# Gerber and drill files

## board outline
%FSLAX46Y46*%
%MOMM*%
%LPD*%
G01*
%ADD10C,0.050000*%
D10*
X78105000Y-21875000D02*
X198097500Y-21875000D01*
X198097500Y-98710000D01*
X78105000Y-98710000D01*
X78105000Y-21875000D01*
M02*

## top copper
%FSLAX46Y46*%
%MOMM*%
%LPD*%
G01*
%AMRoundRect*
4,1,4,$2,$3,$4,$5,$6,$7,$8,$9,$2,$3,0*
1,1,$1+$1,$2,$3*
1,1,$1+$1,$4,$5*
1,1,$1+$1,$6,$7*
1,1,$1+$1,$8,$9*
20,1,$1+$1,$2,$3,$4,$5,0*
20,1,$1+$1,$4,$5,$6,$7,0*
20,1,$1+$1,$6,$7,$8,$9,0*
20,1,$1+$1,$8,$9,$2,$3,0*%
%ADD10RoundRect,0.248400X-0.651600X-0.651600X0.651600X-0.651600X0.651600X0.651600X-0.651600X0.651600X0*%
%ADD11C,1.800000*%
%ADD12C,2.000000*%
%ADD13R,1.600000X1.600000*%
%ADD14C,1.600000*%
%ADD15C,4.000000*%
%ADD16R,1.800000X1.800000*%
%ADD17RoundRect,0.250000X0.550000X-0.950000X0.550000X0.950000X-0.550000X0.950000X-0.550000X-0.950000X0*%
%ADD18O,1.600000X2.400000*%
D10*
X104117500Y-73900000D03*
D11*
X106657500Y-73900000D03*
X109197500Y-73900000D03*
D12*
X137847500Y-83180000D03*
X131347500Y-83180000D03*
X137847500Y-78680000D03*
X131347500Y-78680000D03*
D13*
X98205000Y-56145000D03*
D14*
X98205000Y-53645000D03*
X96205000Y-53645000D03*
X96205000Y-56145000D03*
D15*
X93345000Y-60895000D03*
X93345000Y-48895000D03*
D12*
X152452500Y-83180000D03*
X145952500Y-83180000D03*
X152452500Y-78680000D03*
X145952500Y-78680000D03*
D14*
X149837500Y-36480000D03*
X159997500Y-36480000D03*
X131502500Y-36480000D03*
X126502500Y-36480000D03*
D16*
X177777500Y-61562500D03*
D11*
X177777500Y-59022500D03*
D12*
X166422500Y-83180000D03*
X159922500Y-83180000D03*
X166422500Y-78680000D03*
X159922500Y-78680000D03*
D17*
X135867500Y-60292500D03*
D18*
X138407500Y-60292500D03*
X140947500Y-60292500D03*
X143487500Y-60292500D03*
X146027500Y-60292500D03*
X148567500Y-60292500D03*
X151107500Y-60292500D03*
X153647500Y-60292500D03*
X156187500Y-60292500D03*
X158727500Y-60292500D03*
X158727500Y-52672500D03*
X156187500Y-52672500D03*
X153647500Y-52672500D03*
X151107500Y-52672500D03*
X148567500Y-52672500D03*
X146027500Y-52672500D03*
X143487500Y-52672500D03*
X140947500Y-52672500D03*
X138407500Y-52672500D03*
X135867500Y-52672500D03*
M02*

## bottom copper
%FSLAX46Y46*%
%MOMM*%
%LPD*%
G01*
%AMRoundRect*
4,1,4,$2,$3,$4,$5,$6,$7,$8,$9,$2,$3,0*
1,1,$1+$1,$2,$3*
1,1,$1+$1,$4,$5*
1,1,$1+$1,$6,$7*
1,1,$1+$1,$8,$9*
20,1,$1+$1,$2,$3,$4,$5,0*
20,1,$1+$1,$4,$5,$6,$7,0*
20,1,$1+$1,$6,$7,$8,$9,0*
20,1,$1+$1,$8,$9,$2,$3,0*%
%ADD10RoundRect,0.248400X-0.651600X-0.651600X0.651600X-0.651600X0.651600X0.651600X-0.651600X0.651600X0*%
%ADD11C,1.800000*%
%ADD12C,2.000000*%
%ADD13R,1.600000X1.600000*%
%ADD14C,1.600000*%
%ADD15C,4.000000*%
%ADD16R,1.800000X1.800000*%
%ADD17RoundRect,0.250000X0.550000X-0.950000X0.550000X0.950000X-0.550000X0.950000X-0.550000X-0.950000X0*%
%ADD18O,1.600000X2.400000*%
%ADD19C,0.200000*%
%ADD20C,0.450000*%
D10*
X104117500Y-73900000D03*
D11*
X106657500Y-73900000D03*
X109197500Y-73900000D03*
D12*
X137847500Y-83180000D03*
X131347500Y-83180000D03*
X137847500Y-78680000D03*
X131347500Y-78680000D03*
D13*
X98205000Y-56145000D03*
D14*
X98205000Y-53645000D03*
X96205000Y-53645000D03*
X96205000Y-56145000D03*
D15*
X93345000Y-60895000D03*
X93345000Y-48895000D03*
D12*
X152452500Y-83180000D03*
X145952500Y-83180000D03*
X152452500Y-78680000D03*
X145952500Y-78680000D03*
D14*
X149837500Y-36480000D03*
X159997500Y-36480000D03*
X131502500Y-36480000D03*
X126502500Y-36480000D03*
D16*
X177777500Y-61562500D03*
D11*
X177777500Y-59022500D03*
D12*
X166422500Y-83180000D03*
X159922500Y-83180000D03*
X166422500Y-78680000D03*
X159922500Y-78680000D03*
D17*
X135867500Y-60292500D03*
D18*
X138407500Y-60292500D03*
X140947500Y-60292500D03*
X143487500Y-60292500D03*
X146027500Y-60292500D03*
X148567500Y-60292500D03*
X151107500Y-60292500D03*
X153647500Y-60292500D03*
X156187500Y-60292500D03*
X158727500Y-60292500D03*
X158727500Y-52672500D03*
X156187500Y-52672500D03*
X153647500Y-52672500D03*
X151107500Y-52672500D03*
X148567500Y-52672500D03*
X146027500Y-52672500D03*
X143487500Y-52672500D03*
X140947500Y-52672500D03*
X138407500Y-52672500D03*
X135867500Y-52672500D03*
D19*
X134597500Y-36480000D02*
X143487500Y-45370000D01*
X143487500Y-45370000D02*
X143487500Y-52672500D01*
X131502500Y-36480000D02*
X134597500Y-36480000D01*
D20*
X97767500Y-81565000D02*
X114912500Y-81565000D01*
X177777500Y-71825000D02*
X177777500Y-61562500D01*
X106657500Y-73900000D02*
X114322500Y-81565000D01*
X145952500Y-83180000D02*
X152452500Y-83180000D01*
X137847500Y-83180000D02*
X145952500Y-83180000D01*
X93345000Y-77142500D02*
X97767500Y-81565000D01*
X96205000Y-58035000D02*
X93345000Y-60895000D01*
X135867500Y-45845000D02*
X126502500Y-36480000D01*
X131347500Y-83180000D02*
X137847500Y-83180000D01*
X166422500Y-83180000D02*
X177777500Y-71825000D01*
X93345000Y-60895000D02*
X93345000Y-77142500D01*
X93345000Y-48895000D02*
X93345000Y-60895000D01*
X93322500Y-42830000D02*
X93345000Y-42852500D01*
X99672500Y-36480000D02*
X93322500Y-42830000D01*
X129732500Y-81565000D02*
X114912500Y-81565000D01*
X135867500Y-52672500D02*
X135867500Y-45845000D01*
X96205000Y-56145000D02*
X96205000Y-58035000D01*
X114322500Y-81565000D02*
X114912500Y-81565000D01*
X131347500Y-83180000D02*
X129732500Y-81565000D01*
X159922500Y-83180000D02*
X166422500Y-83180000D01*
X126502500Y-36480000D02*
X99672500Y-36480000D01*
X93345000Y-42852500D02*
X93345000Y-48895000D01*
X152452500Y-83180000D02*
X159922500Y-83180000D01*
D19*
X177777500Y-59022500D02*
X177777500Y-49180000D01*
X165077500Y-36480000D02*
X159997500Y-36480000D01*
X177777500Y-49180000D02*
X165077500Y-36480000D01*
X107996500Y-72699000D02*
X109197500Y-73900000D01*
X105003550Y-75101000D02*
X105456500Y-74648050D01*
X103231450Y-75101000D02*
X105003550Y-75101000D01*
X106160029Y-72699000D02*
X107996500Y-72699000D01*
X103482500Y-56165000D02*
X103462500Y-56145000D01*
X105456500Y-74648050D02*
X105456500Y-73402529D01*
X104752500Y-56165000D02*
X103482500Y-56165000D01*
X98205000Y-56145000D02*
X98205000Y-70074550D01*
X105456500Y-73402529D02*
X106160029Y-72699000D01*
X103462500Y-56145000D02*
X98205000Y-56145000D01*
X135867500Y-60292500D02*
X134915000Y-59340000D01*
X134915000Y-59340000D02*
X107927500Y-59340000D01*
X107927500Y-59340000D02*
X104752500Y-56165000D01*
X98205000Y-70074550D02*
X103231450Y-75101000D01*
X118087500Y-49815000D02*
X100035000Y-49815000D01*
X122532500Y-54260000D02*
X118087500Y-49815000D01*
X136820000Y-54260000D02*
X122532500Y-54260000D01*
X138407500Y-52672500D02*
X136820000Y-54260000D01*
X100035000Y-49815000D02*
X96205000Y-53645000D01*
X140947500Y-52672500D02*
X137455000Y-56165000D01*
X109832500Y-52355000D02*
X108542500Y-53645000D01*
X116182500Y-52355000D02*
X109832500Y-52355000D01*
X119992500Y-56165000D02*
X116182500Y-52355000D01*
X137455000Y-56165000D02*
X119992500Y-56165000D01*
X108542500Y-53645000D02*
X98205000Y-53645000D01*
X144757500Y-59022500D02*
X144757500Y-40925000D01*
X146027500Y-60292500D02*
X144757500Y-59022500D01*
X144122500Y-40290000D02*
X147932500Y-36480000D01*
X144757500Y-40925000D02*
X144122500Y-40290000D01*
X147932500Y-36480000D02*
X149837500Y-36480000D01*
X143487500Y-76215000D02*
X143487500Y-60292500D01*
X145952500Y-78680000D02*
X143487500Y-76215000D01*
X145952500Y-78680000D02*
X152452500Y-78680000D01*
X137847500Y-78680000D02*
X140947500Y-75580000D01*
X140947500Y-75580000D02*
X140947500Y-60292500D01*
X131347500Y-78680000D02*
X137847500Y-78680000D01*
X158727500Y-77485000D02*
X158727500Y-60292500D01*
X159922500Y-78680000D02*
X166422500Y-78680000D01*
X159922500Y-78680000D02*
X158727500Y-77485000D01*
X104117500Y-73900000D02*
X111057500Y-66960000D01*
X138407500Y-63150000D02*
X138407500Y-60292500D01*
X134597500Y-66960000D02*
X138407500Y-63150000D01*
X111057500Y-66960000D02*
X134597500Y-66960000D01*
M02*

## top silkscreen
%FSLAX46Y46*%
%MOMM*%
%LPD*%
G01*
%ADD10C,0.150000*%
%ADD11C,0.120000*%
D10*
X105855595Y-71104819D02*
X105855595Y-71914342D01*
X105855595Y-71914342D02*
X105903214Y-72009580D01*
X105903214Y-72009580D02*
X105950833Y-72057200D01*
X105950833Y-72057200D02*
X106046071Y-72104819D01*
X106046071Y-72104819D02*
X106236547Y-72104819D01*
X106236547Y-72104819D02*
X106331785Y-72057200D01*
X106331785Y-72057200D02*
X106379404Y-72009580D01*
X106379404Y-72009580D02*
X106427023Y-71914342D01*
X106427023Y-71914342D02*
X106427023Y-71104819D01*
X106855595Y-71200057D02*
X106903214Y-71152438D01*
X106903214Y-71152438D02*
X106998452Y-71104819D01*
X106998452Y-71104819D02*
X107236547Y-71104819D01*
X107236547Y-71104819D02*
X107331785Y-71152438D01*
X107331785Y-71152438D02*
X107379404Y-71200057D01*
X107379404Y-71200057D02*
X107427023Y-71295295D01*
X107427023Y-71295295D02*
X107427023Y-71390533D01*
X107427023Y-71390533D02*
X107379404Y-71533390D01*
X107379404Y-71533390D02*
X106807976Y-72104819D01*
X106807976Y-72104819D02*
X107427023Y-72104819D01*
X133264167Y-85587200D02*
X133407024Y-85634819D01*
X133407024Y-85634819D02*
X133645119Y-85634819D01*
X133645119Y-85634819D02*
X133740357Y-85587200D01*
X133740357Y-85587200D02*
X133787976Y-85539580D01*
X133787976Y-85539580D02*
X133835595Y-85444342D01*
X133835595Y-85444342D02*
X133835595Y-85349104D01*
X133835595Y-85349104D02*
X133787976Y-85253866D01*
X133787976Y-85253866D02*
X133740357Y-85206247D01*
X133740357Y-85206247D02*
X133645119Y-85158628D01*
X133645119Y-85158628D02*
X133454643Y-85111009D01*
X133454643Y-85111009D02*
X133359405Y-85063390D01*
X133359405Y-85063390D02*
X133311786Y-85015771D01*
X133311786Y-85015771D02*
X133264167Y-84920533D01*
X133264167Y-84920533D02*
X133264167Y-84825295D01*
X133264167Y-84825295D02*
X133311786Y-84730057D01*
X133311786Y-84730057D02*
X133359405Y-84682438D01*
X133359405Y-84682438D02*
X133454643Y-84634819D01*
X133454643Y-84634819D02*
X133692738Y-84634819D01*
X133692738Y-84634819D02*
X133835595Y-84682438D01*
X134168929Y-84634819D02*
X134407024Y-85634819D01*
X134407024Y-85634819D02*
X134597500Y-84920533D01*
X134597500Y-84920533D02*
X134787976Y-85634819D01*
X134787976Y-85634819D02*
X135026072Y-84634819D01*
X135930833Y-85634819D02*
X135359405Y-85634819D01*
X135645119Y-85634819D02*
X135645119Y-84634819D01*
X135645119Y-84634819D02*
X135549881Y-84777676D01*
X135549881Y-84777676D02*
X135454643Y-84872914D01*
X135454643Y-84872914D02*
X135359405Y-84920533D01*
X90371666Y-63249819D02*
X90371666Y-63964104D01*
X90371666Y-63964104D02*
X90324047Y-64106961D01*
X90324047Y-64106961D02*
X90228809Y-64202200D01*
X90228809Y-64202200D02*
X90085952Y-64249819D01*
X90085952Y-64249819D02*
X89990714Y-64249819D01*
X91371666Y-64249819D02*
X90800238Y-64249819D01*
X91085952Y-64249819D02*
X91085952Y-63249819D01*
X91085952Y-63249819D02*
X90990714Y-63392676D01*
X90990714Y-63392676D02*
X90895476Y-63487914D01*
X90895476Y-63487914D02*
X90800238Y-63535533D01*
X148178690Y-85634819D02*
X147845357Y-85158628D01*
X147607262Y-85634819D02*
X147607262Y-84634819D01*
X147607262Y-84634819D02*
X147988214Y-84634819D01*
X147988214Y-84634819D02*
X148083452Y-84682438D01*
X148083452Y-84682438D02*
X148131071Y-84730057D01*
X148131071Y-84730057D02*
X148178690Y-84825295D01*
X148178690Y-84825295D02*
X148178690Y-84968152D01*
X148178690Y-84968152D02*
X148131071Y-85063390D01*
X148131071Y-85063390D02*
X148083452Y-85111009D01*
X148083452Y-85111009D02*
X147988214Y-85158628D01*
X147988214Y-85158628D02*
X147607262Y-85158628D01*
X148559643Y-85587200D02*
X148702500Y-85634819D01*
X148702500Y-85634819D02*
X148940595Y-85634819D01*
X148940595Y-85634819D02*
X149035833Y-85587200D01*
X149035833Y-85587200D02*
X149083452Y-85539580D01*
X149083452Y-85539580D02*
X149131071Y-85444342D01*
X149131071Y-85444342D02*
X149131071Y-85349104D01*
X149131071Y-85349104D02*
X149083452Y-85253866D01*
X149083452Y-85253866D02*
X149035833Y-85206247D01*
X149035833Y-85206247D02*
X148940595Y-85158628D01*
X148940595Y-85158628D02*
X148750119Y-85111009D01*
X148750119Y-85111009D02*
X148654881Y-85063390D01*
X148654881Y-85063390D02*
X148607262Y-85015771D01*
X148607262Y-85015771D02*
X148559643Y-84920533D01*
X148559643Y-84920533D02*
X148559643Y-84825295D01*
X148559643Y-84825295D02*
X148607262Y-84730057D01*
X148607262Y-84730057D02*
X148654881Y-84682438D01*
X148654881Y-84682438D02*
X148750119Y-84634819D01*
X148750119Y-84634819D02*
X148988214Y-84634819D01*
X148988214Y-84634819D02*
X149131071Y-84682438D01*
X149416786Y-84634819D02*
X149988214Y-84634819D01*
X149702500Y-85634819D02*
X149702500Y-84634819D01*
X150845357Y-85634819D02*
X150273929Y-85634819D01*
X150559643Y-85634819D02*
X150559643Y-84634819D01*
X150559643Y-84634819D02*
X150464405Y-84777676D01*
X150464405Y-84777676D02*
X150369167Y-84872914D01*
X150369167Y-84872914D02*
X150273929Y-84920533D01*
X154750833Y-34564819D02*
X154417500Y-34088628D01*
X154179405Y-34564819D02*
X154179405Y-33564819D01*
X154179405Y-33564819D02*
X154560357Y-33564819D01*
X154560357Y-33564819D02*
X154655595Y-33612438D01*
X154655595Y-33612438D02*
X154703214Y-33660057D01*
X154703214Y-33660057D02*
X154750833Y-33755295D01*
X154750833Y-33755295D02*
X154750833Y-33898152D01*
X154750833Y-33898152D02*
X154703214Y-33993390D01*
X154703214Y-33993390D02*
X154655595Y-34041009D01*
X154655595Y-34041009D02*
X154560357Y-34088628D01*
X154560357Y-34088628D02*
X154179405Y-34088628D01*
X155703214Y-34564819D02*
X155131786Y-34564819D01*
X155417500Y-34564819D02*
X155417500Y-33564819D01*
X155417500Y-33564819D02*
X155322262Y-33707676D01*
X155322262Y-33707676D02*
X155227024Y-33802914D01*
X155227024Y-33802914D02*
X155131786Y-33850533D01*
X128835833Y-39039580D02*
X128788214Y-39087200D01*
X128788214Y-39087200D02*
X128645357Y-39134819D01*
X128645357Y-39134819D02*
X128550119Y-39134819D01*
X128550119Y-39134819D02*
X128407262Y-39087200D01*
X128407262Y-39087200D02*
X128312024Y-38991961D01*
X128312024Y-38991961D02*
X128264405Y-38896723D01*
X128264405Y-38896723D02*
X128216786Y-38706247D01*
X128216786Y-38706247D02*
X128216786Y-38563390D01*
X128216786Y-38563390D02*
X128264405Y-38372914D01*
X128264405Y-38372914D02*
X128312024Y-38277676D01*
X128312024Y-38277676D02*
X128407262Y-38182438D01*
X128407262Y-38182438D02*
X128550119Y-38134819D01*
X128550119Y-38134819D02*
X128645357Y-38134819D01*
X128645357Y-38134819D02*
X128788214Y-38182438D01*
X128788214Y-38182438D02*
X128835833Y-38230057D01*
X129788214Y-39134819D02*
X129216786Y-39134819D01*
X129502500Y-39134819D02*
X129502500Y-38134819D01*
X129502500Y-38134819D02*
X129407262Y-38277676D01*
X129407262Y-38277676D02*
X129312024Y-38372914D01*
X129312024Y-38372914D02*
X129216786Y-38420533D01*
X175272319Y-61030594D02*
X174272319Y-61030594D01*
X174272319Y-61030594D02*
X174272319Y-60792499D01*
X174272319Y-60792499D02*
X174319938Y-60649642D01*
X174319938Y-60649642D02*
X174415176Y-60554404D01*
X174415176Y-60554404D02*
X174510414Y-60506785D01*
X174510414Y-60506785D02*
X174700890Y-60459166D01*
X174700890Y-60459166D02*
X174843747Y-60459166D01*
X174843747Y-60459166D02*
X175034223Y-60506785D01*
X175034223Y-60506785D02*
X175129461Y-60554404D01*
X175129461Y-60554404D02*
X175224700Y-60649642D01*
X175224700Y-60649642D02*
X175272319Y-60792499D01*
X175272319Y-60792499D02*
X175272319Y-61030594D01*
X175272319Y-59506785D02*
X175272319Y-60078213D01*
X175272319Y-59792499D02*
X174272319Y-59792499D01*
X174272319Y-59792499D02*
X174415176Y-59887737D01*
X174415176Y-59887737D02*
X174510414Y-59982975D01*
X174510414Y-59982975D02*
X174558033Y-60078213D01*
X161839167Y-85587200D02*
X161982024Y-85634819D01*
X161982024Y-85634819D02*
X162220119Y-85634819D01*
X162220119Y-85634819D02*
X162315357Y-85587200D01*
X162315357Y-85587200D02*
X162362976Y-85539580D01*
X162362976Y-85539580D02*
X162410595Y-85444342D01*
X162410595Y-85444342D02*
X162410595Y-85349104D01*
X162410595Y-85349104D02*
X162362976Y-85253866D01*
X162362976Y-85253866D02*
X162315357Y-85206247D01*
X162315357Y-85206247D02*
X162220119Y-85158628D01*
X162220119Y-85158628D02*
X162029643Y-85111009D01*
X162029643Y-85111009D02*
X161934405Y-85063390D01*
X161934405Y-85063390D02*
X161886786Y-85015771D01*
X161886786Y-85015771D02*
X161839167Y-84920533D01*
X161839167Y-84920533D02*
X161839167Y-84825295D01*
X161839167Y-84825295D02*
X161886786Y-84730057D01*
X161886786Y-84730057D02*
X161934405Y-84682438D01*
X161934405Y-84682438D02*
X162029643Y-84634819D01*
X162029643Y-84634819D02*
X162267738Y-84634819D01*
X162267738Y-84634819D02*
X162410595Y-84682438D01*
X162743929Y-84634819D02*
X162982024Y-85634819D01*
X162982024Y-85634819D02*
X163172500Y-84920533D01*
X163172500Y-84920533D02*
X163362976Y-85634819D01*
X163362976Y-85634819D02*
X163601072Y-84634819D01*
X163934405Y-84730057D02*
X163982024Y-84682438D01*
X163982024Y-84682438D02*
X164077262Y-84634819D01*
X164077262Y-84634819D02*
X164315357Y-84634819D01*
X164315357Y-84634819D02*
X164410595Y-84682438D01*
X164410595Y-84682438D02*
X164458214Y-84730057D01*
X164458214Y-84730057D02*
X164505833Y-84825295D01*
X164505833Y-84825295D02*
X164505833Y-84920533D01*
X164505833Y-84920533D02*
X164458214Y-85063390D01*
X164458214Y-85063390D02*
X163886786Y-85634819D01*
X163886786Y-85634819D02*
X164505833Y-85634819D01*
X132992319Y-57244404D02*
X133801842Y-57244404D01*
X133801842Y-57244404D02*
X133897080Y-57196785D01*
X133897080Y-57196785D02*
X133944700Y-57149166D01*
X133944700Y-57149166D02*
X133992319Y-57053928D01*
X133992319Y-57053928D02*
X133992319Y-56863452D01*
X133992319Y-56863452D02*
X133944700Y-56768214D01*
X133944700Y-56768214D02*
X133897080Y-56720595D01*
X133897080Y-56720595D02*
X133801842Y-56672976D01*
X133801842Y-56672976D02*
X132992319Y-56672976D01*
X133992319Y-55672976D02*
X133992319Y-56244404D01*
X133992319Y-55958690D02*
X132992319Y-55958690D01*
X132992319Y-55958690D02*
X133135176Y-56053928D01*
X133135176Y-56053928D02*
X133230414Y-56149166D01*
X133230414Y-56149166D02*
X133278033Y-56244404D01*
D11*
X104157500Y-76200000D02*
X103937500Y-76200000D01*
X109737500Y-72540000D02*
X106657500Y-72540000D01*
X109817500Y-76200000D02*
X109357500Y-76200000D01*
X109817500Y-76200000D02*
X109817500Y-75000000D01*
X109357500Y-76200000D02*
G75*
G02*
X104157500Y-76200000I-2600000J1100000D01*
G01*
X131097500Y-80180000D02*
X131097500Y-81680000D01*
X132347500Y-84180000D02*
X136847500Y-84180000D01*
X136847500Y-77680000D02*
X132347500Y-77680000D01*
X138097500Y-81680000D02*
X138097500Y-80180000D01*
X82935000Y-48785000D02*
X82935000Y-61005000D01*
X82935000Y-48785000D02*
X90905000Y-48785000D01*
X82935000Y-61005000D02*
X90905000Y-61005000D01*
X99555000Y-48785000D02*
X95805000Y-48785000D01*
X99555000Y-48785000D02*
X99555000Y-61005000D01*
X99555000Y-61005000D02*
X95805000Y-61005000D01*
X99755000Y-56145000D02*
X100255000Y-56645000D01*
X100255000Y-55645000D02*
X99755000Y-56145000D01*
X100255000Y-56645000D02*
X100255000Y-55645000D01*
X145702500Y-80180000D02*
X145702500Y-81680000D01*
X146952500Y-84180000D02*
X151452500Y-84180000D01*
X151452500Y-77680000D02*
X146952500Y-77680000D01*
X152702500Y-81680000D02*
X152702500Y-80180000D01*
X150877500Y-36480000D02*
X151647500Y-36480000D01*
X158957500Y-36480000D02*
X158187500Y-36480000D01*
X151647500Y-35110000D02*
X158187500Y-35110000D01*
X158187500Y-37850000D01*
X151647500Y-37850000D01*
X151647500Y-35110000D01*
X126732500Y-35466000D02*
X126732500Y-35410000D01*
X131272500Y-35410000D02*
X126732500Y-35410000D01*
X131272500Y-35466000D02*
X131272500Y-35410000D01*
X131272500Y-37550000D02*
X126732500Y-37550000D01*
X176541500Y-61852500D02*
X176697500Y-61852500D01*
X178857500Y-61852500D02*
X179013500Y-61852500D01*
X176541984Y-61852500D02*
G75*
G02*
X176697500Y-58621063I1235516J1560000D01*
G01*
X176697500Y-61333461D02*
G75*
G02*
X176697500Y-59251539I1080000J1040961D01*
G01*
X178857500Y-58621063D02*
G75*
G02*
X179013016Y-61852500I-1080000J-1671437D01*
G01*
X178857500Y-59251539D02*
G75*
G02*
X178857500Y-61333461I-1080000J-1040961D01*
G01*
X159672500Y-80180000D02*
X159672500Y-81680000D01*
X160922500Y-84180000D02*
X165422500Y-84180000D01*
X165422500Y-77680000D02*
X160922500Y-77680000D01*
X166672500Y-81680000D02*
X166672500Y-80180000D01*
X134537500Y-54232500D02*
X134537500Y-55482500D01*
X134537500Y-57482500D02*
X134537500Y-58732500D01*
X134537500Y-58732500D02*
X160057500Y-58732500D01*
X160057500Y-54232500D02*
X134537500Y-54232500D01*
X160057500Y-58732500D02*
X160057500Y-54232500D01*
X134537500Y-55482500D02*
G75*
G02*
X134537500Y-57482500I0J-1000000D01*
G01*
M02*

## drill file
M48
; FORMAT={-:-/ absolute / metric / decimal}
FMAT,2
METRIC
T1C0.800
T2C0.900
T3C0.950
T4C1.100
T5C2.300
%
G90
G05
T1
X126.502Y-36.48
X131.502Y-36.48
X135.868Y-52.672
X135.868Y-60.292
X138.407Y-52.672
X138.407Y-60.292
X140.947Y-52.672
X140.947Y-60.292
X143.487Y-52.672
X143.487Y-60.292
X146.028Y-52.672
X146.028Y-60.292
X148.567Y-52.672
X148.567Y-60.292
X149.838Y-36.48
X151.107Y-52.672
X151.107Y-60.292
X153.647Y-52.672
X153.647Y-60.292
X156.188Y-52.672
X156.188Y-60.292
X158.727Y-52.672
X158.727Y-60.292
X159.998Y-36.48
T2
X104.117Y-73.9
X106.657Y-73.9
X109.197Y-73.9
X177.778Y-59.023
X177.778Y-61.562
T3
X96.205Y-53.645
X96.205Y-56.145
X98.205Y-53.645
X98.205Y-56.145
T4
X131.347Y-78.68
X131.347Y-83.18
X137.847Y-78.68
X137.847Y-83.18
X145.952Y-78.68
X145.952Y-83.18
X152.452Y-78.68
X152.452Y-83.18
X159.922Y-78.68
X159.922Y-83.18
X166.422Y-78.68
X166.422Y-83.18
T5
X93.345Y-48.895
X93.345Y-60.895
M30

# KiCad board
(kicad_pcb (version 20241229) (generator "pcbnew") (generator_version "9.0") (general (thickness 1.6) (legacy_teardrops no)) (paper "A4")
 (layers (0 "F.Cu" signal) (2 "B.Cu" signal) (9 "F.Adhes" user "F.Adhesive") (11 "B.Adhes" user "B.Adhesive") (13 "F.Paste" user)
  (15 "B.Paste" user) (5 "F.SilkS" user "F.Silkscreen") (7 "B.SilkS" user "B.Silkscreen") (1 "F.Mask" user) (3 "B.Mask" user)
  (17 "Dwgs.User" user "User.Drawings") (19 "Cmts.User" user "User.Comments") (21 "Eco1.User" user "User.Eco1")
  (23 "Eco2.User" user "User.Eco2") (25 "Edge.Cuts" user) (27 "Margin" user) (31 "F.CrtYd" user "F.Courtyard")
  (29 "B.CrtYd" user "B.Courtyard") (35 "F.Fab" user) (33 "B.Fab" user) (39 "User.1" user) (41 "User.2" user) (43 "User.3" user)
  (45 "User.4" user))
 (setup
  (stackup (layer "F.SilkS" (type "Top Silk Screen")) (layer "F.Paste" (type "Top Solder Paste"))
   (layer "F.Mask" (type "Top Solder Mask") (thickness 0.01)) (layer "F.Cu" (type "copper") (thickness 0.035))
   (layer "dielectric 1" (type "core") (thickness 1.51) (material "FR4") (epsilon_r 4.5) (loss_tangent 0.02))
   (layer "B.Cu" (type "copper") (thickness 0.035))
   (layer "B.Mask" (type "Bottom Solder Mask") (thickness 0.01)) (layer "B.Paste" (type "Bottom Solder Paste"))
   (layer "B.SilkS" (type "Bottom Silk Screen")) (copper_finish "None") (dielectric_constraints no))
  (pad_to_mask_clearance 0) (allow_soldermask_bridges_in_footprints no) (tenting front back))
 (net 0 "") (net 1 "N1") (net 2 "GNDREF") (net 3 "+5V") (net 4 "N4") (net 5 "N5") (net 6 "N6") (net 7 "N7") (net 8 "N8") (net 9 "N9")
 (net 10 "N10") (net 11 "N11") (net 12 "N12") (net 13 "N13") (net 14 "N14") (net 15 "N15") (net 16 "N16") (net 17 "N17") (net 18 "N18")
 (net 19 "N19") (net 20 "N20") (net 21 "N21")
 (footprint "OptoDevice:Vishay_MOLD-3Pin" (layer "F.Cu") (at 104.1175 73.9)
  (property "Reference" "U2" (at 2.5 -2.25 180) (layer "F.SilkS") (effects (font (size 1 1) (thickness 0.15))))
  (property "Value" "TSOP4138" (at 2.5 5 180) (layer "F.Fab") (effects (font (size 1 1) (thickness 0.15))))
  (fp_line (start 0.04 2.3) (end -0.18 2.3) (stroke (width 0.12) (type solid)) (layer "F.SilkS"))
  (fp_line (start 5.62 -1.36) (end 2.54 -1.36) (stroke (width 0.12) (type solid)) (layer "F.SilkS"))
  (fp_line (start 5.7 2.3) (end 5.24 2.3) (stroke (width 0.12) (type solid)) (layer "F.SilkS"))
  (fp_line (start 5.7 2.3) (end 5.7 1.1) (stroke (width 0.12) (type solid)) (layer "F.SilkS"))
  (fp_arc (start 5.24 2.3) (mid 2.64 4.023119) (end 0.04 2.3) (stroke (width 0.12) (type solid)) (layer "F.SilkS"))
  (pad "1" thru_hole roundrect (at 0 0) (size 1.8 1.8) (drill 0.9) (layers "*.Cu" "*.Mask") (remove_unused_layers no)
   (roundrect_rratio 0.138) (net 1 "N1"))
  (pad "2" thru_hole circle (at 2.54 0) (size 1.8 1.8) (drill 0.9) (layers "*.Cu" "*.Mask") (remove_unused_layers no) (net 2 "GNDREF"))
  (pad "3" thru_hole circle (at 5.08 0) (size 1.8 1.8) (drill 0.9) (layers "*.Cu" "*.Mask") (remove_unused_layers no) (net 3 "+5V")))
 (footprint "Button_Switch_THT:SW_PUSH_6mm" (layer "F.Cu") (at 137.8475 83.18 180)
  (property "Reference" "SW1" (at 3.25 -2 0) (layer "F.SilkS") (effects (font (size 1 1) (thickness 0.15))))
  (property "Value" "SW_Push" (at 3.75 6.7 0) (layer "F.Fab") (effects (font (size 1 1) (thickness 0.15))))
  (fp_line (start 6.75 3) (end 6.75 1.5) (stroke (width 0.12) (type solid)) (layer "F.SilkS"))
  (fp_line (start 5.5 -1) (end 1 -1) (stroke (width 0.12) (type solid)) (layer "F.SilkS"))
  (fp_line (start 1 5.5) (end 5.5 5.5) (stroke (width 0.12) (type solid)) (layer "F.SilkS"))
  (fp_line (start -0.25 1.5) (end -0.25 3) (stroke (width 0.12) (type solid)) (layer "F.SilkS"))
  (pad "1" thru_hole circle (at 0 0 270) (size 2 2) (drill 1.1) (layers "*.Cu" "*.Mask") (remove_unused_layers no) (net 2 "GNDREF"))
  (pad "1" thru_hole circle (at 6.5 0 270) (size 2 2) (drill 1.1) (layers "*.Cu" "*.Mask") (remove_unused_layers no) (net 2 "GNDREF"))
  (pad "2" thru_hole circle (at 0 4.5 270) (size 2 2) (drill 1.1) (layers "*.Cu" "*.Mask") (remove_unused_layers no) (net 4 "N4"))
  (pad "2" thru_hole circle (at 6.5 4.5 270) (size 2 2) (drill 1.1) (layers "*.Cu" "*.Mask") (remove_unused_layers no) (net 4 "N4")))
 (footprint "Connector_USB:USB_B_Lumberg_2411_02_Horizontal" (layer "F.Cu") (at 98.205 56.145 180)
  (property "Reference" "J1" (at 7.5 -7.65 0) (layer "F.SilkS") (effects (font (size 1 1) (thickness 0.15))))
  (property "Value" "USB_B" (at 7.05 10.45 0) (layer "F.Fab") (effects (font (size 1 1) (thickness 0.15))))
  (fp_line (start 15.27 7.36) (end 15.27 -4.86) (stroke (width 0.12) (type solid)) (layer "F.SilkS"))
  (fp_line (start 15.27 7.36) (end 7.3 7.36) (stroke (width 0.12) (type solid)) (layer "F.SilkS"))
  (fp_line (start 15.27 -4.86) (end 7.3 -4.86) (stroke (width 0.12) (type solid)) (layer "F.SilkS"))
  (fp_line (start -1.35 7.36) (end 2.4 7.36) (stroke (width 0.12) (type solid)) (layer "F.SilkS"))
  (fp_line (start -1.35 7.36) (end -1.35 -4.86) (stroke (width 0.12) (type solid)) (layer "F.SilkS"))
  (fp_line (start -1.35 -4.86) (end 2.4 -4.86) (stroke (width 0.12) (type solid)) (layer "F.SilkS"))
  (fp_line (start -1.55 0) (end -2.05 -0.5) (stroke (width 0.12) (type solid)) (layer "F.SilkS"))
  (fp_line (start -2.05 0.5) (end -1.55 0) (stroke (width 0.12) (type solid)) (layer "F.SilkS"))
  (fp_line (start -2.05 -0.5) (end -2.05 0.5) (stroke (width 0.12) (type solid)) (layer "F.SilkS"))
  (pad "1" thru_hole rect (at 0 0 270) (size 1.6 1.6) (drill 0.95) (layers "*.Cu" "*.Mask") (remove_unused_layers no) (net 3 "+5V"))
  (pad "2" thru_hole circle (at 0 2.5 270) (size 1.6 1.6) (drill 0.95) (layers "*.Cu" "*.Mask") (remove_unused_layers no) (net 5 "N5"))
  (pad "3" thru_hole circle (at 2 2.5 270) (size 1.6 1.6) (drill 0.95) (layers "*.Cu" "*.Mask") (remove_unused_layers no) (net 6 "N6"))
  (pad "4" thru_hole circle (at 2 0 270) (size 1.6 1.6) (drill 0.95) (layers "*.Cu" "*.Mask") (remove_unused_layers no) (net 2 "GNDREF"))
  (pad "5" thru_hole circle (at 4.86 -4.75 270) (size 4 4) (drill 2.3) (layers "*.Cu" "*.Mask") (remove_unused_layers no) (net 2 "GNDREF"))
  (pad "5" thru_hole circle (at 4.86 7.25 270) (size 4 4) (drill 2.3) (layers "*.Cu" "*.Mask") (remove_unused_layers no) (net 2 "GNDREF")))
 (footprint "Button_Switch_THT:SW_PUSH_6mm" (layer "F.Cu") (at 152.4525 83.18 180)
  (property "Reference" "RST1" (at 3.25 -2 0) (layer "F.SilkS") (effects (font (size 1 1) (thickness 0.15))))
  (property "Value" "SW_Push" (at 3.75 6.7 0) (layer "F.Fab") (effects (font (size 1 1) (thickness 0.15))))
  (fp_line (start 6.75 3) (end 6.75 1.5) (stroke (width 0.12) (type solid)) (layer "F.SilkS"))
  (fp_line (start 5.5 -1) (end 1 -1) (stroke (width 0.12) (type solid)) (layer "F.SilkS"))
  (fp_line (start 1 5.5) (end 5.5 5.5) (stroke (width 0.12) (type solid)) (layer "F.SilkS"))
  (fp_line (start -0.25 1.5) (end -0.25 3) (stroke (width 0.12) (type solid)) (layer "F.SilkS"))
  (pad "1" thru_hole circle (at 0 0 270) (size 2 2) (drill 1.1) (layers "*.Cu" "*.Mask") (remove_unused_layers no) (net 2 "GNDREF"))
  (pad "1" thru_hole circle (at 6.5 0 270) (size 2 2) (drill 1.1) (layers "*.Cu" "*.Mask") (remove_unused_layers no) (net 2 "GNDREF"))
  (pad "2" thru_hole circle (at 0 4.5 270) (size 2 2) (drill 1.1) (layers "*.Cu" "*.Mask") (remove_unused_layers no) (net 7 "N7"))
  (pad "2" thru_hole circle (at 6.5 4.5 270) (size 2 2) (drill 1.1) (layers "*.Cu" "*.Mask") (remove_unused_layers no) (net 7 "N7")))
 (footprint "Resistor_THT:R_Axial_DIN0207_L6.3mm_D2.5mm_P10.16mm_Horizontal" (layer "F.Cu") (at 149.8375 36.48)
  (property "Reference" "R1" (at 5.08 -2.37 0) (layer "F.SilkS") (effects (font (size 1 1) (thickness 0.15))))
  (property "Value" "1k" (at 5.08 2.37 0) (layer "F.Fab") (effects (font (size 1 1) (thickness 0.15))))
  (fp_line (start 1.04 0) (end 1.81 0) (stroke (width 0.12) (type solid)) (layer "F.SilkS"))
  (fp_line (start 9.12 0) (end 8.35 0) (stroke (width 0.12) (type solid)) (layer "F.SilkS"))
  (fp_rect (start 1.81 -1.37) (end 8.35 1.37) (stroke (width 0.12) (type solid)) (fill no) (layer "F.SilkS"))
  (pad "1" thru_hole circle (at 0 0) (size 1.6 1.6) (drill 0.8) (layers "*.Cu" "*.Mask") (remove_unused_layers no) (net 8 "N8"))
  (pad "2" thru_hole circle (at 10.16 0) (size 1.6 1.6) (drill 0.8) (layers "*.Cu" "*.Mask") (remove_unused_layers no) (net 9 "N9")))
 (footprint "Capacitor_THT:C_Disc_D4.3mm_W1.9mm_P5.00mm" (layer "F.Cu") (at 131.5025 36.48 180)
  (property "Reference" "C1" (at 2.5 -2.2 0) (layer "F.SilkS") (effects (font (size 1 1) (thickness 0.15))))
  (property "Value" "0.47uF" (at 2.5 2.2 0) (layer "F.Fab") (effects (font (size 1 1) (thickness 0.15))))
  (fp_line (start 4.77 1.014) (end 4.77 1.07) (stroke (width 0.12) (type solid)) (layer "F.SilkS"))
  (fp_line (start 0.23 1.07) (end 4.77 1.07) (stroke (width 0.12) (type solid)) (layer "F.SilkS"))
  (fp_line (start 0.23 1.014) (end 0.23 1.07) (stroke (width 0.12) (type solid)) (layer "F.SilkS"))
  (fp_line (start 0.23 -1.07) (end 4.77 -1.07) (stroke (width 0.12) (type solid)) (layer "F.SilkS"))
  (pad "1" thru_hole circle (at 0 0 180) (size 1.6 1.6) (drill 0.8) (layers "*.Cu" "*.Mask") (remove_unused_layers no) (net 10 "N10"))
  (pad "2" thru_hole circle (at 5 0 180) (size 1.6 1.6) (drill 0.8) (layers "*.Cu" "*.Mask") (remove_unused_layers no) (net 2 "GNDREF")))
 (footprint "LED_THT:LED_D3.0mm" (layer "F.Cu") (at 177.7775 61.5625 90)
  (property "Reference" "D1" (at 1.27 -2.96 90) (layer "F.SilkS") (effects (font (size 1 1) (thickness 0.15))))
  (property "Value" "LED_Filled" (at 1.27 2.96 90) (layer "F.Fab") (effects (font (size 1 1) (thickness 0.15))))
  (fp_line (start -0.29 -1.236) (end -0.29 -1.08) (stroke (width 0.12) (type solid)) (layer "F.SilkS"))
  (fp_line (start -0.29 1.08) (end -0.29 1.236) (stroke (width 0.12) (type solid)) (layer "F.SilkS"))
  (fp_arc (start -0.29 -1.235516) (mid 1.36566 -1.987699) (end 2.941437 -1.08) (stroke (width 0.12) (type solid)) (layer "F.SilkS"))
  (fp_arc (start 0.229039 -1.08) (mid 1.27 -1.5) (end 2.310961 -1.08) (stroke (width 0.12) (type solid)) (layer "F.SilkS"))
  (fp_arc (start 2.941437 1.08) (mid 1.36566 1.987699) (end -0.29 1.235516) (stroke (width 0.12) (type solid)) (layer "F.SilkS"))
  (fp_arc (start 2.310961 1.08) (mid 1.27 1.5) (end 0.229039 1.08) (stroke (width 0.12) (type solid)) (layer "F.SilkS"))
  (pad "1" thru_hole rect (at 0 0 90) (size 1.8 1.8) (drill 0.9) (layers "*.Cu" "*.Mask") (remove_unused_layers no) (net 2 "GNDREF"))
  (pad "2" thru_hole circle (at 2.54 0 90) (size 1.8 1.8) (drill 0.9) (layers "*.Cu" "*.Mask") (remove_unused_layers no) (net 9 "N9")))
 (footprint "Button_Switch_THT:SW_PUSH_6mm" (layer "F.Cu") (at 166.4225 83.18 180)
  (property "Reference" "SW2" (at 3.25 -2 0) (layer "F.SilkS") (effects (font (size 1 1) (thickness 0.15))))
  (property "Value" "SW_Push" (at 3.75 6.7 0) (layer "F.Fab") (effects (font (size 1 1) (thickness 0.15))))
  (fp_line (start 6.75 3) (end 6.75 1.5) (stroke (width 0.12) (type solid)) (layer "F.SilkS"))
  (fp_line (start 5.5 -1) (end 1 -1) (stroke (width 0.12) (type solid)) (layer "F.SilkS"))
  (fp_line (start 1 5.5) (end 5.5 5.5) (stroke (width 0.12) (type solid)) (layer "F.SilkS"))
  (fp_line (start -0.25 1.5) (end -0.25 3) (stroke (width 0.12) (type solid)) (layer "F.SilkS"))
  (pad "1" thru_hole circle (at 0 0 270) (size 2 2) (drill 1.1) (layers "*.Cu" "*.Mask") (remove_unused_layers no) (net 2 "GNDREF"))
  (pad "1" thru_hole circle (at 6.5 0 270) (size 2 2) (drill 1.1) (layers "*.Cu" "*.Mask") (remove_unused_layers no) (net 2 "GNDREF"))
  (pad "2" thru_hole circle (at 0 4.5 270) (size 2 2) (drill 1.1) (layers "*.Cu" "*.Mask") (remove_unused_layers no) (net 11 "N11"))
  (pad "2" thru_hole circle (at 6.5 4.5 270) (size 2 2) (drill 1.1) (layers "*.Cu" "*.Mask") (remove_unused_layers no) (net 11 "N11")))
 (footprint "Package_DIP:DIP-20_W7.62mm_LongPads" (layer "F.Cu") (at 135.8675 60.2925 90)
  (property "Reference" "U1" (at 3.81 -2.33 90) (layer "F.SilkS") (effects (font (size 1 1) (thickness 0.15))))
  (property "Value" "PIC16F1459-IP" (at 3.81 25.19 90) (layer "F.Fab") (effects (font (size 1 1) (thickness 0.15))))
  (fp_line (start 6.06 -1.33) (end 4.81 -1.33) (stroke (width 0.12) (type solid)) (layer "F.SilkS"))
  (fp_line (start 2.81 -1.33) (end 1.56 -1.33) (stroke (width 0.12) (type solid)) (layer "F.SilkS"))
  (fp_line (start 1.56 -1.33) (end 1.56 24.19) (stroke (width 0.12) (type solid)) (layer "F.SilkS"))
  (fp_line (start 6.06 24.19) (end 6.06 -1.33) (stroke (width 0.12) (type solid)) (layer "F.SilkS"))
  (fp_line (start 1.56 24.19) (end 6.06 24.19) (stroke (width 0.12) (type solid)) (layer "F.SilkS"))
  (fp_arc (start 4.81 -1.33) (mid 3.81 -0.33) (end 2.81 -1.33) (stroke (width 0.12) (type solid)) (layer "F.SilkS"))
  (pad "1" thru_hole roundrect (at 0 0 90) (size 2.4 1.6) (drill 0.8) (layers "*.Cu" "*.Mask") (remove_unused_layers no)
   (roundrect_rratio 0.15625) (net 3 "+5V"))
  (pad "2" thru_hole oval (at 0 2.54 90) (size 2.4 1.6) (drill 0.8) (layers "*.Cu" "*.Mask") (remove_unused_layers no) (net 1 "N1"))
  (pad "3" thru_hole oval (at 0 5.08 90) (size 2.4 1.6) (drill 0.8) (layers "*.Cu" "*.Mask") (remove_unused_layers no) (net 4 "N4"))
  (pad "4" thru_hole oval (at 0 7.62 90) (size 2.4 1.6) (drill 0.8) (layers "*.Cu" "*.Mask") (remove_unused_layers no) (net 7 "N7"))
  (pad "5" thru_hole oval (at 0 10.16 90) (size 2.4 1.6) (drill 0.8) (layers "*.Cu" "*.Mask") (remove_unused_layers no) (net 8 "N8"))
  (pad "6" thru_hole oval (at 0 12.7 90) (size 2.4 1.6) (drill 0.8) (layers "*.Cu" "*.Mask") (remove_unused_layers no) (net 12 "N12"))
  (pad "7" thru_hole oval (at 0 15.24 90) (size 2.4 1.6) (drill 0.8) (layers "*.Cu" "*.Mask") (remove_unused_layers no) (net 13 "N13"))
  (pad "8" thru_hole oval (at 0 17.78 90) (size 2.4 1.6) (drill 0.8) (layers "*.Cu" "*.Mask") (remove_unused_layers no) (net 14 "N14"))
  (pad "9" thru_hole oval (at 0 20.32 90) (size 2.4 1.6) (drill 0.8) (layers "*.Cu" "*.Mask") (remove_unused_layers no) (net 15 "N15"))
  (pad "10" thru_hole oval (at 0 22.86 90) (size 2.4 1.6) (drill 0.8) (layers "*.Cu" "*.Mask") (remove_unused_layers no) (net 11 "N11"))
  (pad "11" thru_hole oval (at 7.62 22.86 90) (size 2.4 1.6) (drill 0.8) (layers "*.Cu" "*.Mask") (remove_unused_layers no) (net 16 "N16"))
  (pad "12" thru_hole oval (at 7.62 20.32 90) (size 2.4 1.6) (drill 0.8) (layers "*.Cu" "*.Mask") (remove_unused_layers no) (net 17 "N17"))
  (pad "13" thru_hole oval (at 7.62 17.78 90) (size 2.4 1.6) (drill 0.8) (layers "*.Cu" "*.Mask") (remove_unused_layers no) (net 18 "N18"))
  (pad "14" thru_hole oval (at 7.62 15.24 90) (size 2.4 1.6) (drill 0.8) (layers "*.Cu" "*.Mask") (remove_unused_layers no) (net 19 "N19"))
  (pad "15" thru_hole oval (at 7.62 12.7 90) (size 2.4 1.6) (drill 0.8) (layers "*.Cu" "*.Mask") (remove_unused_layers no) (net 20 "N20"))
  (pad "16" thru_hole oval (at 7.62 10.16 90) (size 2.4 1.6) (drill 0.8) (layers "*.Cu" "*.Mask") (remove_unused_layers no) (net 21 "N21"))
  (pad "17" thru_hole oval (at 7.62 7.62 90) (size 2.4 1.6) (drill 0.8) (layers "*.Cu" "*.Mask") (remove_unused_layers no) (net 10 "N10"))
  (pad "18" thru_hole oval (at 7.62 5.08 90) (size 2.4 1.6) (drill 0.8) (layers "*.Cu" "*.Mask") (remove_unused_layers no) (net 5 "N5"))
  (pad "19" thru_hole oval (at 7.62 2.54 90) (size 2.4 1.6) (drill 0.8) (layers "*.Cu" "*.Mask") (remove_unused_layers no) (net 6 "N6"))
  (pad "20" thru_hole oval (at 7.62 0 90) (size 2.4 1.6) (drill 0.8) (layers "*.Cu" "*.Mask") (remove_unused_layers no) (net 2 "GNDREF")))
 (gr_rect (start 78.105 21.875) (end 198.0975 98.71) (stroke (width 0.05) (type default)) (fill no) (layer "Edge.Cuts"))
 (segment (start 134.5975 36.48) (end 143.4875 45.37) (width 0.2) (layer "B.Cu") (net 10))
 (segment (start 143.4875 45.37) (end 143.4875 52.6725) (width 0.2) (layer "B.Cu") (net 10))
 (segment (start 131.5025 36.48) (end 134.5975 36.48) (width 0.2) (layer "B.Cu") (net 10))
 (segment (start 97.7675 81.565) (end 114.9125 81.565) (width 0.45) (layer "B.Cu") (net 2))
 (segment (start 177.7775 71.825) (end 177.7775 61.5625) (width 0.45) (layer "B.Cu") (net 2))
 (segment (start 106.6575 73.9) (end 114.3225 81.565) (width 0.45) (layer "B.Cu") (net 2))
 (segment (start 145.9525 83.18) (end 152.4525 83.18) (width 0.45) (layer "B.Cu") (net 2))
 (segment (start 137.8475 83.18) (end 145.9525 83.18) (width 0.45) (layer "B.Cu") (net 2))
 (segment (start 93.345 77.1425) (end 97.7675 81.565) (width 0.45) (layer "B.Cu") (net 2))
 (segment (start 96.205 58.035) (end 93.345 60.895) (width 0.45) (layer "B.Cu") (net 2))
 (segment (start 135.8675 45.845) (end 126.5025 36.48) (width 0.45) (layer "B.Cu") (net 2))
 (segment (start 131.3475 83.18) (end 137.8475 83.18) (width 0.45) (layer "B.Cu") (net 2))
 (segment (start 166.4225 83.18) (end 177.7775 71.825) (width 0.45) (layer "B.Cu") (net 2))
 (segment (start 93.345 60.895) (end 93.345 77.1425) (width 0.45) (layer "B.Cu") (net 2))
 (segment (start 93.345 48.895) (end 93.345 60.895) (width 0.45) (layer "B.Cu") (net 2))
 (segment (start 93.3225 42.83) (end 93.345 42.8525) (width 0.45) (layer "B.Cu") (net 2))
 (segment (start 99.6725 36.48) (end 93.3225 42.83) (width 0.45) (layer "B.Cu") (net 2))
 (segment (start 129.7325 81.565) (end 114.9125 81.565) (width 0.45) (layer "B.Cu") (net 2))
 (segment (start 135.8675 52.6725) (end 135.8675 45.845) (width 0.45) (layer "B.Cu") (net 2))
 (segment (start 96.205 56.145) (end 96.205 58.035) (width 0.45) (layer "B.Cu") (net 2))
 (segment (start 114.3225 81.565) (end 114.9125 81.565) (width 0.45) (layer "B.Cu") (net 2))
 (segment (start 131.3475 83.18) (end 129.7325 81.565) (width 0.45) (layer "B.Cu") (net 2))
 (segment (start 159.9225 83.18) (end 166.4225 83.18) (width 0.45) (layer "B.Cu") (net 2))
 (segment (start 126.5025 36.48) (end 99.6725 36.48) (width 0.45) (layer "B.Cu") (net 2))
 (segment (start 93.345 42.8525) (end 93.345 48.895) (width 0.45) (layer "B.Cu") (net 2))
 (segment (start 152.4525 83.18) (end 159.9225 83.18) (width 0.45) (layer "B.Cu") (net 2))
 (segment (start 177.7775 59.0225) (end 177.7775 49.18) (width 0.2) (layer "B.Cu") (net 9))
 (segment (start 165.0775 36.48) (end 159.9975 36.48) (width 0.2) (layer "B.Cu") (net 9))
 (segment (start 177.7775 49.18) (end 165.0775 36.48) (width 0.2) (layer "B.Cu") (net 9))
 (segment (start 107.9965 72.699) (end 109.1975 73.9) (width 0.2) (layer "B.Cu") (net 3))
 (segment (start 105.00355 75.101) (end 105.4565 74.64805) (width 0.2) (layer "B.Cu") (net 3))
 (segment (start 103.23145 75.101) (end 105.00355 75.101) (width 0.2) (layer "B.Cu") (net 3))
 (segment (start 106.160029 72.699) (end 107.9965 72.699) (width 0.2) (layer "B.Cu") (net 3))
 (segment (start 103.4825 56.165) (end 103.4625 56.145) (width 0.2) (layer "B.Cu") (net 3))
 (segment (start 105.4565 74.64805) (end 105.4565 73.402529) (width 0.2) (layer "B.Cu") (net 3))
 (segment (start 104.7525 56.165) (end 103.4825 56.165) (width 0.2) (layer "B.Cu") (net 3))
 (segment (start 98.205 56.145) (end 98.205 70.07455) (width 0.2) (layer "B.Cu") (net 3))
 (segment (start 105.4565 73.402529) (end 106.160029 72.699) (width 0.2) (layer "B.Cu") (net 3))
 (segment (start 103.4625 56.145) (end 98.205 56.145) (width 0.2) (layer "B.Cu") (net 3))
 (segment (start 135.8675 60.2925) (end 134.915 59.34) (width 0.2) (layer "B.Cu") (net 3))
 (segment (start 134.915 59.34) (end 107.9275 59.34) (width 0.2) (layer "B.Cu") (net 3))
 (segment (start 107.9275 59.34) (end 104.7525 56.165) (width 0.2) (layer "B.Cu") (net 3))
 (segment (start 98.205 70.07455) (end 103.23145 75.101) (width 0.2) (layer "B.Cu") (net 3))
 (segment (start 118.0875 49.815) (end 100.035 49.815) (width 0.2) (layer "B.Cu") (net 6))
 (segment (start 122.5325 54.26) (end 118.0875 49.815) (width 0.2) (layer "B.Cu") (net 6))
 (segment (start 136.82 54.26) (end 122.5325 54.26) (width 0.2) (layer "B.Cu") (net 6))
 (segment (start 138.4075 52.6725) (end 136.82 54.26) (width 0.2) (layer "B.Cu") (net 6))
 (segment (start 100.035 49.815) (end 96.205 53.645) (width 0.2) (layer "B.Cu") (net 6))
 (segment (start 140.9475 52.6725) (end 137.455 56.165) (width 0.2) (layer "B.Cu") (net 5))
 (segment (start 109.8325 52.355) (end 108.5425 53.645) (width 0.2) (layer "B.Cu") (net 5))
 (segment (start 116.1825 52.355) (end 109.8325 52.355) (width 0.2) (layer "B.Cu") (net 5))
 (segment (start 119.9925 56.165) (end 116.1825 52.355) (width 0.2) (layer "B.Cu") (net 5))
 (segment (start 137.455 56.165) (end 119.9925 56.165) (width 0.2) (layer "B.Cu") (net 5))
 (segment (start 108.5425 53.645) (end 98.205 53.645) (width 0.2) (layer "B.Cu") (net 5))
 (segment (start 144.7575 59.0225) (end 144.7575 40.925) (width 0.2) (layer "B.Cu") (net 8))
 (segment (start 146.0275 60.2925) (end 144.7575 59.0225) (width 0.2) (layer "B.Cu") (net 8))
 (segment (start 144.1225 40.29) (end 147.9325 36.48) (width 0.2) (layer "B.Cu") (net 8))
 (segment (start 144.7575 40.925) (end 144.1225 40.29) (width 0.2) (layer "B.Cu") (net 8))
 (segment (start 147.9325 36.48) (end 149.8375 36.48) (width 0.2) (layer "B.Cu") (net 8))
 (segment (start 143.4875 76.215) (end 143.4875 60.2925) (width 0.2) (layer "B.Cu") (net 7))
 (segment (start 145.9525 78.68) (end 143.4875 76.215) (width 0.2) (layer "B.Cu") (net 7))
 (segment (start 145.9525 78.68) (end 152.4525 78.68) (width 0.2) (layer "B.Cu") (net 7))
 (segment (start 137.8475 78.68) (end 140.9475 75.58) (width 0.2) (layer "B.Cu") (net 4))
 (segment (start 140.9475 75.58) (end 140.9475 60.2925) (width 0.2) (layer "B.Cu") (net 4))
 (segment (start 131.3475 78.68) (end 137.8475 78.68) (width 0.2) (layer "B.Cu") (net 4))
 (segment (start 158.7275 77.485) (end 158.7275 60.2925) (width 0.2) (layer "B.Cu") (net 11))
 (segment (start 159.9225 78.68) (end 166.4225 78.68) (width 0.2) (layer "B.Cu") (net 11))
 (segment (start 159.9225 78.68) (end 158.7275 77.485) (width 0.2) (layer "B.Cu") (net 11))
 (segment (start 104.1175 73.9) (end 111.0575 66.96) (width 0.2) (layer "B.Cu") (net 1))
 (segment (start 138.4075 63.15) (end 138.4075 60.2925) (width 0.2) (layer "B.Cu") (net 1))
 (segment (start 134.5975 66.96) (end 138.4075 63.15) (width 0.2) (layer "B.Cu") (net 1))
 (segment (start 111.0575 66.96) (end 134.5975 66.96) (width 0.2) (layer "B.Cu") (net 1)))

